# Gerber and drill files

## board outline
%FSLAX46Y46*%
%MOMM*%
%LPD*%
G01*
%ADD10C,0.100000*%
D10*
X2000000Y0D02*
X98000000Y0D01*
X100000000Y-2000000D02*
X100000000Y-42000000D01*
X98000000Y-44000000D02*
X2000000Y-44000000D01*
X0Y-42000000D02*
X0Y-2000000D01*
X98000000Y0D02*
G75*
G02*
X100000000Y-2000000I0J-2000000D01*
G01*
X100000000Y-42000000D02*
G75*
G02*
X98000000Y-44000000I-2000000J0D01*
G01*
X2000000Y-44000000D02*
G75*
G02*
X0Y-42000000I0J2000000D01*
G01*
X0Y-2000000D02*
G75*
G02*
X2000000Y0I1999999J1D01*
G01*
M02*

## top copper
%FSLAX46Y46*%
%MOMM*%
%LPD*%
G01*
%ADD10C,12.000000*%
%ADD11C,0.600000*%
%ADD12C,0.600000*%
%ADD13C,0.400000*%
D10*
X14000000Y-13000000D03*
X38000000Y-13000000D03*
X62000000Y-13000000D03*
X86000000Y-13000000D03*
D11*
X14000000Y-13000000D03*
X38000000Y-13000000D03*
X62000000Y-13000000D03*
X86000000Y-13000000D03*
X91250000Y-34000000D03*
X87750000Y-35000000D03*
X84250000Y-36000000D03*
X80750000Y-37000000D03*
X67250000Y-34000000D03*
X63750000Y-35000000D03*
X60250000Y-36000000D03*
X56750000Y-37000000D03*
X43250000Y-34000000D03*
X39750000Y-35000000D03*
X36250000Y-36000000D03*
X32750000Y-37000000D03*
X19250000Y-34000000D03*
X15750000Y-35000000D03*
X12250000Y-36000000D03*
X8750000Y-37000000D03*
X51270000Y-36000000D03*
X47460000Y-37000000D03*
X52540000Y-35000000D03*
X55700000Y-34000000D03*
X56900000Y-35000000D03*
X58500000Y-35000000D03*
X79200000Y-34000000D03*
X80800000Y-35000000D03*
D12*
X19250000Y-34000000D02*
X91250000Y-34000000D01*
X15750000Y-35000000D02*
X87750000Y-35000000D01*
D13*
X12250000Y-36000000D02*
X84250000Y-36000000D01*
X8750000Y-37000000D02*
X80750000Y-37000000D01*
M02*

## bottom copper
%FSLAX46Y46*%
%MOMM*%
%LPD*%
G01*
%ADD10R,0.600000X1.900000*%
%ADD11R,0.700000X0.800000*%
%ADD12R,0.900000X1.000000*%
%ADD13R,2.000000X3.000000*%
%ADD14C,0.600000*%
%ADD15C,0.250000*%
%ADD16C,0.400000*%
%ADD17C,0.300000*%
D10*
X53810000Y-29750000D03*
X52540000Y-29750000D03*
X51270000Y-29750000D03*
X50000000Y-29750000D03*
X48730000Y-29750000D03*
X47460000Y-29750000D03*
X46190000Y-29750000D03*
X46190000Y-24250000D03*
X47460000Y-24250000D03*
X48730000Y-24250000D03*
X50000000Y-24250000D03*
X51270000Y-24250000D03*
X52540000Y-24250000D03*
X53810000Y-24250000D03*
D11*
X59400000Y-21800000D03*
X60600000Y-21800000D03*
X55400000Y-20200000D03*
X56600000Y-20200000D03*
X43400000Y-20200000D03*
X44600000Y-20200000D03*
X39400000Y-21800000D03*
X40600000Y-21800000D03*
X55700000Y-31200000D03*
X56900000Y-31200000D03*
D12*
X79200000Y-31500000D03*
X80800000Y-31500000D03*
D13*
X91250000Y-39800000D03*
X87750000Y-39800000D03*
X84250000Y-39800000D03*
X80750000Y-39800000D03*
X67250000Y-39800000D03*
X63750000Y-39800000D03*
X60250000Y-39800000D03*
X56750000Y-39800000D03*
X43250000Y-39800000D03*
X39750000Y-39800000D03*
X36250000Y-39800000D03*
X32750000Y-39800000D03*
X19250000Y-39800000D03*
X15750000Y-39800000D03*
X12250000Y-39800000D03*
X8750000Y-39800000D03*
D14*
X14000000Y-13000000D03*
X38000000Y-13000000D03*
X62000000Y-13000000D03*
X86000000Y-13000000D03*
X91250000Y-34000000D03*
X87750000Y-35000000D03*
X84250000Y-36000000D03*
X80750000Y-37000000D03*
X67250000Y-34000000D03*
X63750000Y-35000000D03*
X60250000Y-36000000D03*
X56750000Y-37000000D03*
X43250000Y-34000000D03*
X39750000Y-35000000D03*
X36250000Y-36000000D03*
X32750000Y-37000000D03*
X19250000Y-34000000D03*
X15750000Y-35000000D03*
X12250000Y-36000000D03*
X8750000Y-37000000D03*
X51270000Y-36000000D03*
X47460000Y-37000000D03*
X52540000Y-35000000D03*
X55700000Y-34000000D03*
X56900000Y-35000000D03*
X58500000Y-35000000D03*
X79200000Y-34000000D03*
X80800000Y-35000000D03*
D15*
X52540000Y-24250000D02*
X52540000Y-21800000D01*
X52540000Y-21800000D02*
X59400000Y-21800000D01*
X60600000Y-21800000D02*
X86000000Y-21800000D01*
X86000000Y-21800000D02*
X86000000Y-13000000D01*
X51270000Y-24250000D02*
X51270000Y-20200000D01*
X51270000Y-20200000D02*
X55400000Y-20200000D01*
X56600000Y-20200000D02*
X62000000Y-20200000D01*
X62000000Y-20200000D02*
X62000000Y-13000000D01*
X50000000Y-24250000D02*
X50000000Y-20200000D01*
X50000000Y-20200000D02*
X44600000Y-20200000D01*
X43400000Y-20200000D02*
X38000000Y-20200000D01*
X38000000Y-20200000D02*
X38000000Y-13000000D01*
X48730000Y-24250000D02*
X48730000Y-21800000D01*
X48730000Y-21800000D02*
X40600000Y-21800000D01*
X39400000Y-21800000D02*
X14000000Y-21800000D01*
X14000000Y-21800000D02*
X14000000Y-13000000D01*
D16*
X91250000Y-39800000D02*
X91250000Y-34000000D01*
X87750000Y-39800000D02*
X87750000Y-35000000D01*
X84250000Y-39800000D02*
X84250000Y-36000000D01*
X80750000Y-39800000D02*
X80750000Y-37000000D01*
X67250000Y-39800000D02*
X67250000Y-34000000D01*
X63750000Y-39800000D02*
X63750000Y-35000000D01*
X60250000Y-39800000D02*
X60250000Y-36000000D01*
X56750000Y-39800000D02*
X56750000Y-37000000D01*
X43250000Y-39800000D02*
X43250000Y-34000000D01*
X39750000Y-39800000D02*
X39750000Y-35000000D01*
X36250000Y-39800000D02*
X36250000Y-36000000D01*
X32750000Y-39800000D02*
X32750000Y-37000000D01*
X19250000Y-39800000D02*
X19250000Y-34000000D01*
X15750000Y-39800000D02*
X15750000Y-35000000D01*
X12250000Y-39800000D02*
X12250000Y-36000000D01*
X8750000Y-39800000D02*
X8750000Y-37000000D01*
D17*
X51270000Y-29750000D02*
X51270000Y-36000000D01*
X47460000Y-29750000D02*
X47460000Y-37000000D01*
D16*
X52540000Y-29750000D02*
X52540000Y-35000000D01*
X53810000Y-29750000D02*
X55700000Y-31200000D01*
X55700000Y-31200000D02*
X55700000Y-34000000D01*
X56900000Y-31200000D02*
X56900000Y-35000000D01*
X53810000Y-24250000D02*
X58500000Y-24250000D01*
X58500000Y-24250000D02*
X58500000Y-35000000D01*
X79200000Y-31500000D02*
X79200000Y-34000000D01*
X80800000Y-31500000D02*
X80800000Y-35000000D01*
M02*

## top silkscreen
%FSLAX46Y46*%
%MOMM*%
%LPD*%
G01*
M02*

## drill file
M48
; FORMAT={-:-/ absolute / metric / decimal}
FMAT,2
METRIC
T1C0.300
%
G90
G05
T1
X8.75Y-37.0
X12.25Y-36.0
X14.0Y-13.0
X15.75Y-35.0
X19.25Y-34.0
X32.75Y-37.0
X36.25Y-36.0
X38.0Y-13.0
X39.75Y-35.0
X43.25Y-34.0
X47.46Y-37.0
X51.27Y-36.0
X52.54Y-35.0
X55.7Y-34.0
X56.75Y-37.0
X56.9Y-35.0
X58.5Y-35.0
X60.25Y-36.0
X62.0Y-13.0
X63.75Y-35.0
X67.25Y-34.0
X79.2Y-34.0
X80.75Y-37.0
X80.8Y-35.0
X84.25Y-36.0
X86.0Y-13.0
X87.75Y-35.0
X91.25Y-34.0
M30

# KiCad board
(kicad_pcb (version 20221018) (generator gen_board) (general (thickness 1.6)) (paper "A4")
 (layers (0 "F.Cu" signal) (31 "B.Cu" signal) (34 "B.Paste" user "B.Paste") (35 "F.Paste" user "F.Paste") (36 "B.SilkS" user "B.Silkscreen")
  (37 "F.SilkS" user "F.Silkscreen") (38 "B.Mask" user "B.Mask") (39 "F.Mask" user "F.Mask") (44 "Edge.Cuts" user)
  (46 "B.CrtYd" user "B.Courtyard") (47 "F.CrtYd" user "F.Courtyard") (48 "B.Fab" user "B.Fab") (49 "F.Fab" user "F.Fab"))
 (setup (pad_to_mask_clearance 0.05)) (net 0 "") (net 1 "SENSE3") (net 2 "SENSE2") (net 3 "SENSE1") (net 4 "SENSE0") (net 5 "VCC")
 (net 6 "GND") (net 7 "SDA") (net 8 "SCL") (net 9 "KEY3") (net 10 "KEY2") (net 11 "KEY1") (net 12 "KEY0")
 (gr_line (start 2.0 0) (end 98.0 0) (stroke (width 0.1) (type default)) (layer "Edge.Cuts"))
 (gr_line (start 100.0 2.0) (end 100.0 42.0) (stroke (width 0.1) (type default)) (layer "Edge.Cuts"))
 (gr_line (start 98.0 44.0) (end 2.0 44.0) (stroke (width 0.1) (type default)) (layer "Edge.Cuts"))
 (gr_line (start 0 42.0) (end 0 2.0) (stroke (width 0.1) (type default)) (layer "Edge.Cuts"))
 (gr_arc (start 98.0 0) (mid 99.4142136 0.5857864) (end 100.0 2.0) (stroke (width 0.1) (type default)) (layer "Edge.Cuts"))
 (gr_arc (start 100.0 42.0) (mid 99.4142136 43.4142136) (end 98.0 44.0) (stroke (width 0.1) (type default)) (layer "Edge.Cuts"))
 (gr_arc (start 2.0 44.0) (mid 0.5857864 43.4142136) (end 0 42.0) (stroke (width 0.1) (type default)) (layer "Edge.Cuts"))
 (gr_arc (start 0 2.0) (mid 0.5857864 0.5857864) (end 2.0 0) (stroke (width 0.1) (type default)) (layer "Edge.Cuts"))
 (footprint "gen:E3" (layer "F.Cu") (at 14.0 13.0)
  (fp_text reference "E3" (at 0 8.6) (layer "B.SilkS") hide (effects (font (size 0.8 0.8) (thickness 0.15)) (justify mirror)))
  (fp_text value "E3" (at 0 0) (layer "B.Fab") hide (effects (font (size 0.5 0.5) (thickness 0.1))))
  (pad "1" smd circle (at 0 0) (size 12.0 12.0) (layers "F.Cu") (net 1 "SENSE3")))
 (via (at 14.0 13.0) (size 0.6) (drill 0.3) (layers "F.Cu" "B.Cu") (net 1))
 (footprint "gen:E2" (layer "F.Cu") (at 38.0 13.0)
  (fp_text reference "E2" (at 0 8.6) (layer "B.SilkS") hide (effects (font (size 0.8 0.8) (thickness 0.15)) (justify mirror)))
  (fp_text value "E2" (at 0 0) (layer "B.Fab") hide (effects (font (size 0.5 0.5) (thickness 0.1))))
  (pad "1" smd circle (at 0 0) (size 12.0 12.0) (layers "F.Cu") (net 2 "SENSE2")))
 (via (at 38.0 13.0) (size 0.6) (drill 0.3) (layers "F.Cu" "B.Cu") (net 2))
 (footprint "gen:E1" (layer "F.Cu") (at 62.0 13.0)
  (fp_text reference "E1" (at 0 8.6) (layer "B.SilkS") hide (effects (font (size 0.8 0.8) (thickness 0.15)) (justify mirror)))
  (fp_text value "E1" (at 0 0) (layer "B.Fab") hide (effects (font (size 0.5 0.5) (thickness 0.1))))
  (pad "1" smd circle (at 0 0) (size 12.0 12.0) (layers "F.Cu") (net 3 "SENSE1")))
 (via (at 62.0 13.0) (size 0.6) (drill 0.3) (layers "F.Cu" "B.Cu") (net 3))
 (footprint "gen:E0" (layer "F.Cu") (at 86.0 13.0)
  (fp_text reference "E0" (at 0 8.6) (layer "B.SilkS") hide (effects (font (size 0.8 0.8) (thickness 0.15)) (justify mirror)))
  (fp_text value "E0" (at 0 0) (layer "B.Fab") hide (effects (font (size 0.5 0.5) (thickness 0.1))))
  (pad "1" smd circle (at 0 0) (size 12.0 12.0) (layers "F.Cu") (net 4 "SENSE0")))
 (via (at 86.0 13.0) (size 0.6) (drill 0.3) (layers "F.Cu" "B.Cu") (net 4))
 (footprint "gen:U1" (layer "B.Cu") (at 50.0 27.0)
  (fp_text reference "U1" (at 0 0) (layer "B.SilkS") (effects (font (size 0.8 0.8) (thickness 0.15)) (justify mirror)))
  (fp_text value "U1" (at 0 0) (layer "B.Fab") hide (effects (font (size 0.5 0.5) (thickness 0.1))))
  (pad "1" smd rect (at 3.8100000000000023 2.75) (size 0.6 1.9) (layers "B.Cu" "B.Mask" "B.Paste") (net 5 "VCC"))
  (pad "2" smd rect (at 2.539999999999999 2.75) (size 0.6 1.9) (layers "B.Cu" "B.Mask" "B.Paste") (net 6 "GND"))
  (pad "3" smd rect (at 1.2700000000000031 2.75) (size 0.6 1.9) (layers "B.Cu" "B.Mask" "B.Paste") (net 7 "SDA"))
  (pad "4" smd rect (at 0.0 2.75) (size 0.6 1.9) (layers "B.Cu" "B.Mask" "B.Paste"))
  (pad "5" smd rect (at -1.269999999999996 2.75) (size 0.6 1.9) (layers "B.Cu" "B.Mask" "B.Paste"))
  (pad "6" smd rect (at -2.539999999999999 2.75) (size 0.6 1.9) (layers "B.Cu" "B.Mask" "B.Paste") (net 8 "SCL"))
  (pad "7" smd rect (at -3.809999999999995 2.75) (size 0.6 1.9) (layers "B.Cu" "B.Mask" "B.Paste"))
  (pad "8" smd rect (at -3.8100000000000023 -2.75) (size 0.6 1.9) (layers "B.Cu" "B.Mask" "B.Paste"))
  (pad "9" smd rect (at -2.539999999999999 -2.75) (size 0.6 1.9) (layers "B.Cu" "B.Mask" "B.Paste"))
  (pad "10" smd rect (at -1.2700000000000031 -2.75) (size 0.6 1.9) (layers "B.Cu" "B.Mask" "B.Paste") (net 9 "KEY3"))
  (pad "11" smd rect (at 0.0 -2.75) (size 0.6 1.9) (layers "B.Cu" "B.Mask" "B.Paste") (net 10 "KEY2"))
  (pad "12" smd rect (at 1.269999999999996 -2.75) (size 0.6 1.9) (layers "B.Cu" "B.Mask" "B.Paste") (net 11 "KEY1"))
  (pad "13" smd rect (at 2.539999999999999 -2.75) (size 0.6 1.9) (layers "B.Cu" "B.Mask" "B.Paste") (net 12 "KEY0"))
  (pad "14" smd rect (at 3.809999999999995 -2.75) (size 0.6 1.9) (layers "B.Cu" "B.Mask" "B.Paste") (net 6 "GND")))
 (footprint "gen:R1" (layer "B.Cu") (at 60.0 21.8)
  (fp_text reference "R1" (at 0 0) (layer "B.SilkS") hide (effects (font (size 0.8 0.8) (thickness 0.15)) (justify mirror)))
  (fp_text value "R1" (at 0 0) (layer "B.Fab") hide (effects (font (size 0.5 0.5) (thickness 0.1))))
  (pad "1" smd rect (at -0.6 0) (size 0.7 0.8) (layers "B.Cu" "B.Mask" "B.Paste") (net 12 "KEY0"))
  (pad "2" smd rect (at 0.6 0) (size 0.7 0.8) (layers "B.Cu" "B.Mask" "B.Paste") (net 4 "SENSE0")))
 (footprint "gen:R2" (layer "B.Cu") (at 56.0 20.2)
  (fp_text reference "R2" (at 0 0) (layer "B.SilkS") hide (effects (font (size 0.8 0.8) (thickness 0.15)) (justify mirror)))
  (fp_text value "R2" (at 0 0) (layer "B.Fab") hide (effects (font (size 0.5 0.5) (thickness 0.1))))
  (pad "1" smd rect (at -0.6 0) (size 0.7 0.8) (layers "B.Cu" "B.Mask" "B.Paste") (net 11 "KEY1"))
  (pad "2" smd rect (at 0.6 0) (size 0.7 0.8) (layers "B.Cu" "B.Mask" "B.Paste") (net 3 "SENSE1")))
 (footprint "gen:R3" (layer "B.Cu") (at 44.0 20.2)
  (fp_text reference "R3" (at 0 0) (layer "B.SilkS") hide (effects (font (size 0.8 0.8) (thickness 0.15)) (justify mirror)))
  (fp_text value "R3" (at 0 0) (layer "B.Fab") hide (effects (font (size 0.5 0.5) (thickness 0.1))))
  (pad "1" smd rect (at -0.6 0) (size 0.7 0.8) (layers "B.Cu" "B.Mask" "B.Paste") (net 2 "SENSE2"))
  (pad "2" smd rect (at 0.6 0) (size 0.7 0.8) (layers "B.Cu" "B.Mask" "B.Paste") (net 10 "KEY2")))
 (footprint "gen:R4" (layer "B.Cu") (at 40.0 21.8)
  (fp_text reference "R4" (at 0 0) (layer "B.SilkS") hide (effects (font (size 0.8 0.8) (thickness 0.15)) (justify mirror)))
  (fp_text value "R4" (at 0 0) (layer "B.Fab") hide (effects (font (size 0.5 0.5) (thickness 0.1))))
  (pad "1" smd rect (at -0.6 0) (size 0.7 0.8) (layers "B.Cu" "B.Mask" "B.Paste") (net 1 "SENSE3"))
  (pad "2" smd rect (at 0.6 0) (size 0.7 0.8) (layers "B.Cu" "B.Mask" "B.Paste") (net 9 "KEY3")))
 (segment (start 52.54 24.25) (end 52.54 21.8) (width 0.25) (layer "B.Cu") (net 12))
 (segment (start 52.54 21.8) (end 59.4 21.8) (width 0.25) (layer "B.Cu") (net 12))
 (segment (start 60.6 21.8) (end 86 21.8) (width 0.25) (layer "B.Cu") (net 4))
 (segment (start 86 21.8) (end 86 13.0) (width 0.25) (layer "B.Cu") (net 4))
 (segment (start 51.269999999999996 24.25) (end 51.269999999999996 20.2) (width 0.25) (layer "B.Cu") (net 11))
 (segment (start 51.269999999999996 20.2) (end 55.4 20.2) (width 0.25) (layer "B.Cu") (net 11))
 (segment (start 56.6 20.2) (end 62 20.2) (width 0.25) (layer "B.Cu") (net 3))
 (segment (start 62 20.2) (end 62 13.0) (width 0.25) (layer "B.Cu") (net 3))
 (segment (start 50.0 24.25) (end 50.0 20.2) (width 0.25) (layer "B.Cu") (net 10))
 (segment (start 50.0 20.2) (end 44.6 20.2) (width 0.25) (layer "B.Cu") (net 10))
 (segment (start 43.4 20.2) (end 38 20.2) (width 0.25) (layer "B.Cu") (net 2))
 (segment (start 38 20.2) (end 38 13.0) (width 0.25) (layer "B.Cu") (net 2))
 (segment (start 48.73 24.25) (end 48.73 21.8) (width 0.25) (layer "B.Cu") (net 9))
 (segment (start 48.73 21.8) (end 40.6 21.8) (width 0.25) (layer "B.Cu") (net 9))
 (segment (start 39.4 21.8) (end 14 21.8) (width 0.25) (layer "B.Cu") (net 1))
 (segment (start 14 21.8) (end 14 13.0) (width 0.25) (layer "B.Cu") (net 1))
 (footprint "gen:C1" (layer "B.Cu") (at 56.3 31.2)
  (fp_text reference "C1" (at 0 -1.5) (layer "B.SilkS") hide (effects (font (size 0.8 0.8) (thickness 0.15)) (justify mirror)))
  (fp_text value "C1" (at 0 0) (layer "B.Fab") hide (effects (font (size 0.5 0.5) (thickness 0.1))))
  (pad "1" smd rect (at -0.6 0) (size 0.7 0.8) (layers "B.Cu" "B.Mask" "B.Paste") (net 5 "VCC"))
  (pad "2" smd rect (at 0.6 0) (size 0.7 0.8) (layers "B.Cu" "B.Mask" "B.Paste") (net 6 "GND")))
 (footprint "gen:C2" (layer "B.Cu") (at 80.0 31.5)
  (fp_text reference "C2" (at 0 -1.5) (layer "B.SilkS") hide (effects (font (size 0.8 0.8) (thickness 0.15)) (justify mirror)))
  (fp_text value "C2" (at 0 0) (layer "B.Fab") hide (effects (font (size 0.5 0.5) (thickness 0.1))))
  (pad "1" smd rect (at -0.8 0) (size 0.9 1.0) (layers "B.Cu" "B.Mask" "B.Paste") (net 5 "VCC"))
  (pad "2" smd rect (at 0.8 0) (size 0.9 1.0) (layers "B.Cu" "B.Mask" "B.Paste") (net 6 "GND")))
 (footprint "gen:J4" (layer "B.Cu") (at 86.0 39.8)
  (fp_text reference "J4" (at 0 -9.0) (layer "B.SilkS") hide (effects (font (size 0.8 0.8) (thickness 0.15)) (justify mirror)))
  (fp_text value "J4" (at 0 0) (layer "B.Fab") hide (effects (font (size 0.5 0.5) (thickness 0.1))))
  (pad "1" smd rect (at 5.25 0) (size 2.0 3.0) (layers "B.Cu" "B.Mask") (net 5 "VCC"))
  (pad "2" smd rect (at 1.75 0) (size 2.0 3.0) (layers "B.Cu" "B.Mask") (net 6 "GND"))
  (pad "3" smd rect (at -1.75 0) (size 2.0 3.0) (layers "B.Cu" "B.Mask") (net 7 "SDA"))
  (pad "4" smd rect (at -5.25 0) (size 2.0 3.0) (layers "B.Cu" "B.Mask") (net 8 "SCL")))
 (via (at 91.25 34.0) (size 0.6) (drill 0.3) (layers "F.Cu" "B.Cu") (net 5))
 (segment (start 91.25 39.8) (end 91.25 34.0) (width 0.4) (layer "B.Cu") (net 5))
 (via (at 87.75 35.0) (size 0.6) (drill 0.3) (layers "F.Cu" "B.Cu") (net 6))
 (segment (start 87.75 39.8) (end 87.75 35.0) (width 0.4) (layer "B.Cu") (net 6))
 (via (at 84.25 36.0) (size 0.6) (drill 0.3) (layers "F.Cu" "B.Cu") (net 7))
 (segment (start 84.25 39.8) (end 84.25 36.0) (width 0.4) (layer "B.Cu") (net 7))
 (via (at 80.75 37.0) (size 0.6) (drill 0.3) (layers "F.Cu" "B.Cu") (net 8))
 (segment (start 80.75 39.8) (end 80.75 37.0) (width 0.4) (layer "B.Cu") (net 8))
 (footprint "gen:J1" (layer "B.Cu") (at 62.0 39.8)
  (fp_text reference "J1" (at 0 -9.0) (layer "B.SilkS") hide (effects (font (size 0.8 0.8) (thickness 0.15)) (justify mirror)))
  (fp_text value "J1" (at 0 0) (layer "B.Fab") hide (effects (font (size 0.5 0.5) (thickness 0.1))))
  (pad "1" smd rect (at 5.25 0) (size 2.0 3.0) (layers "B.Cu" "B.Mask") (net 5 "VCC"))
  (pad "2" smd rect (at 1.75 0) (size 2.0 3.0) (layers "B.Cu" "B.Mask") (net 6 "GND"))
  (pad "3" smd rect (at -1.75 0) (size 2.0 3.0) (layers "B.Cu" "B.Mask") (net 7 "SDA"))
  (pad "4" smd rect (at -5.25 0) (size 2.0 3.0) (layers "B.Cu" "B.Mask") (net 8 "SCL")))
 (via (at 67.25 34.0) (size 0.6) (drill 0.3) (layers "F.Cu" "B.Cu") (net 5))
 (segment (start 67.25 39.8) (end 67.25 34.0) (width 0.4) (layer "B.Cu") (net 5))
 (via (at 63.75 35.0) (size 0.6) (drill 0.3) (layers "F.Cu" "B.Cu") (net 6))
 (segment (start 63.75 39.8) (end 63.75 35.0) (width 0.4) (layer "B.Cu") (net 6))
 (via (at 60.25 36.0) (size 0.6) (drill 0.3) (layers "F.Cu" "B.Cu") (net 7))
 (segment (start 60.25 39.8) (end 60.25 36.0) (width 0.4) (layer "B.Cu") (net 7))
 (via (at 56.75 37.0) (size 0.6) (drill 0.3) (layers "F.Cu" "B.Cu") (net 8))
 (segment (start 56.75 39.8) (end 56.75 37.0) (width 0.4) (layer "B.Cu") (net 8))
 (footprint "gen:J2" (layer "B.Cu") (at 38.0 39.8)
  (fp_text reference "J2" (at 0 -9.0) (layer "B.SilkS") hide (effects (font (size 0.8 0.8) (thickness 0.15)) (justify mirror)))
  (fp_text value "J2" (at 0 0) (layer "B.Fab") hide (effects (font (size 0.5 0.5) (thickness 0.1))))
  (pad "1" smd rect (at 5.25 0) (size 2.0 3.0) (layers "B.Cu" "B.Mask") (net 5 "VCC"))
  (pad "2" smd rect (at 1.75 0) (size 2.0 3.0) (layers "B.Cu" "B.Mask") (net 6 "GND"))
  (pad "3" smd rect (at -1.75 0) (size 2.0 3.0) (layers "B.Cu" "B.Mask") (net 7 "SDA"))
  (pad "4" smd rect (at -5.25 0) (size 2.0 3.0) (layers "B.Cu" "B.Mask") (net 8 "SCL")))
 (via (at 43.25 34.0) (size 0.6) (drill 0.3) (layers "F.Cu" "B.Cu") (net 5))
 (segment (start 43.25 39.8) (end 43.25 34.0) (width 0.4) (layer "B.Cu") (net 5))
 (via (at 39.75 35.0) (size 0.6) (drill 0.3) (layers "F.Cu" "B.Cu") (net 6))
 (segment (start 39.75 39.8) (end 39.75 35.0) (width 0.4) (layer "B.Cu") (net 6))
 (via (at 36.25 36.0) (size 0.6) (drill 0.3) (layers "F.Cu" "B.Cu") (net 7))
 (segment (start 36.25 39.8) (end 36.25 36.0) (width 0.4) (layer "B.Cu") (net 7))
 (via (at 32.75 37.0) (size 0.6) (drill 0.3) (layers "F.Cu" "B.Cu") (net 8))
 (segment (start 32.75 39.8) (end 32.75 37.0) (width 0.4) (layer "B.Cu") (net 8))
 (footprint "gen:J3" (layer "B.Cu") (at 14.0 39.8)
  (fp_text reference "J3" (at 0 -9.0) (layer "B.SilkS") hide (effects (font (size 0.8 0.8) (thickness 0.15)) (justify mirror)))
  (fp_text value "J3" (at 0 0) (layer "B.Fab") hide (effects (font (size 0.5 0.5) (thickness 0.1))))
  (pad "1" smd rect (at 5.25 0) (size 2.0 3.0) (layers "B.Cu" "B.Mask") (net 5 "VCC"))
  (pad "2" smd rect (at 1.75 0) (size 2.0 3.0) (layers "B.Cu" "B.Mask") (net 6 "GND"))
  (pad "3" smd rect (at -1.75 0) (size 2.0 3.0) (layers "B.Cu" "B.Mask") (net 7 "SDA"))
  (pad "4" smd rect (at -5.25 0) (size 2.0 3.0) (layers "B.Cu" "B.Mask") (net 8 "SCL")))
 (via (at 19.25 34.0) (size 0.6) (drill 0.3) (layers "F.Cu" "B.Cu") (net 5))
 (segment (start 19.25 39.8) (end 19.25 34.0) (width 0.4) (layer "B.Cu") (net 5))
 (via (at 15.75 35.0) (size 0.6) (drill 0.3) (layers "F.Cu" "B.Cu") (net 6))
 (segment (start 15.75 39.8) (end 15.75 35.0) (width 0.4) (layer "B.Cu") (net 6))
 (via (at 12.25 36.0) (size 0.6) (drill 0.3) (layers "F.Cu" "B.Cu") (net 7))
 (segment (start 12.25 39.8) (end 12.25 36.0) (width 0.4) (layer "B.Cu") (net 7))
 (via (at 8.75 37.0) (size 0.6) (drill 0.3) (layers "F.Cu" "B.Cu") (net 8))
 (segment (start 8.75 39.8) (end 8.75 37.0) (width 0.4) (layer "B.Cu") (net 8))
 (segment (start 19.25 34.0) (end 91.25 34.0) (width 0.6) (layer "F.Cu") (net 5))
 (segment (start 15.75 35.0) (end 87.75 35.0) (width 0.6) (layer "F.Cu") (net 6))
 (segment (start 12.25 36.0) (end 84.25 36.0) (width 0.4) (layer "F.Cu") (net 7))
 (segment (start 8.75 37.0) (end 80.75 37.0) (width 0.4) (layer "F.Cu") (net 8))
 (segment (start 51.27 29.75) (end 51.27 36.0) (width 0.3) (layer "B.Cu") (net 7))
 (via (at 51.27 36.0) (size 0.6) (drill 0.3) (layers "F.Cu" "B.Cu") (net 7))
 (segment (start 47.46 29.75) (end 47.46 37.0) (width 0.3) (layer "B.Cu") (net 8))
 (via (at 47.46 37.0) (size 0.6) (drill 0.3) (layers "F.Cu" "B.Cu") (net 8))
 (segment (start 52.54 29.75) (end 52.54 35.0) (width 0.4) (layer "B.Cu") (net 6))
 (via (at 52.54 35.0) (size 0.6) (drill 0.3) (layers "F.Cu" "B.Cu") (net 6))
 (segment (start 53.81 29.75) (end 55.7 31.2) (width 0.4) (layer "B.Cu") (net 5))
 (segment (start 55.7 31.2) (end 55.7 34.0) (width 0.4) (layer "B.Cu") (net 5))
 (via (at 55.7 34.0) (size 0.6) (drill 0.3) (layers "F.Cu" "B.Cu") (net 5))
 (segment (start 56.9 31.2) (end 56.9 35.0) (width 0.4) (layer "B.Cu") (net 6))
 (via (at 56.9 35.0) (size 0.6) (drill 0.3) (layers "F.Cu" "B.Cu") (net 6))
 (segment (start 53.809999999999995 24.25) (end 58.5 24.25) (width 0.4) (layer "B.Cu") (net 6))
 (segment (start 58.5 24.25) (end 58.5 35.0) (width 0.4) (layer "B.Cu") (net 6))
 (via (at 58.5 35.0) (size 0.6) (drill 0.3) (layers "F.Cu" "B.Cu") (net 6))
 (segment (start 79.2 31.5) (end 79.2 34.0) (width 0.4) (layer "B.Cu") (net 5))
 (via (at 79.2 34.0) (size 0.6) (drill 0.3) (layers "F.Cu" "B.Cu") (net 5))
 (segment (start 80.8 31.5) (end 80.8 35.0) (width 0.4) (layer "B.Cu") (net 6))
 (via (at 80.8 35.0) (size 0.6) (drill 0.3) (layers "F.Cu" "B.Cu") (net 6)))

